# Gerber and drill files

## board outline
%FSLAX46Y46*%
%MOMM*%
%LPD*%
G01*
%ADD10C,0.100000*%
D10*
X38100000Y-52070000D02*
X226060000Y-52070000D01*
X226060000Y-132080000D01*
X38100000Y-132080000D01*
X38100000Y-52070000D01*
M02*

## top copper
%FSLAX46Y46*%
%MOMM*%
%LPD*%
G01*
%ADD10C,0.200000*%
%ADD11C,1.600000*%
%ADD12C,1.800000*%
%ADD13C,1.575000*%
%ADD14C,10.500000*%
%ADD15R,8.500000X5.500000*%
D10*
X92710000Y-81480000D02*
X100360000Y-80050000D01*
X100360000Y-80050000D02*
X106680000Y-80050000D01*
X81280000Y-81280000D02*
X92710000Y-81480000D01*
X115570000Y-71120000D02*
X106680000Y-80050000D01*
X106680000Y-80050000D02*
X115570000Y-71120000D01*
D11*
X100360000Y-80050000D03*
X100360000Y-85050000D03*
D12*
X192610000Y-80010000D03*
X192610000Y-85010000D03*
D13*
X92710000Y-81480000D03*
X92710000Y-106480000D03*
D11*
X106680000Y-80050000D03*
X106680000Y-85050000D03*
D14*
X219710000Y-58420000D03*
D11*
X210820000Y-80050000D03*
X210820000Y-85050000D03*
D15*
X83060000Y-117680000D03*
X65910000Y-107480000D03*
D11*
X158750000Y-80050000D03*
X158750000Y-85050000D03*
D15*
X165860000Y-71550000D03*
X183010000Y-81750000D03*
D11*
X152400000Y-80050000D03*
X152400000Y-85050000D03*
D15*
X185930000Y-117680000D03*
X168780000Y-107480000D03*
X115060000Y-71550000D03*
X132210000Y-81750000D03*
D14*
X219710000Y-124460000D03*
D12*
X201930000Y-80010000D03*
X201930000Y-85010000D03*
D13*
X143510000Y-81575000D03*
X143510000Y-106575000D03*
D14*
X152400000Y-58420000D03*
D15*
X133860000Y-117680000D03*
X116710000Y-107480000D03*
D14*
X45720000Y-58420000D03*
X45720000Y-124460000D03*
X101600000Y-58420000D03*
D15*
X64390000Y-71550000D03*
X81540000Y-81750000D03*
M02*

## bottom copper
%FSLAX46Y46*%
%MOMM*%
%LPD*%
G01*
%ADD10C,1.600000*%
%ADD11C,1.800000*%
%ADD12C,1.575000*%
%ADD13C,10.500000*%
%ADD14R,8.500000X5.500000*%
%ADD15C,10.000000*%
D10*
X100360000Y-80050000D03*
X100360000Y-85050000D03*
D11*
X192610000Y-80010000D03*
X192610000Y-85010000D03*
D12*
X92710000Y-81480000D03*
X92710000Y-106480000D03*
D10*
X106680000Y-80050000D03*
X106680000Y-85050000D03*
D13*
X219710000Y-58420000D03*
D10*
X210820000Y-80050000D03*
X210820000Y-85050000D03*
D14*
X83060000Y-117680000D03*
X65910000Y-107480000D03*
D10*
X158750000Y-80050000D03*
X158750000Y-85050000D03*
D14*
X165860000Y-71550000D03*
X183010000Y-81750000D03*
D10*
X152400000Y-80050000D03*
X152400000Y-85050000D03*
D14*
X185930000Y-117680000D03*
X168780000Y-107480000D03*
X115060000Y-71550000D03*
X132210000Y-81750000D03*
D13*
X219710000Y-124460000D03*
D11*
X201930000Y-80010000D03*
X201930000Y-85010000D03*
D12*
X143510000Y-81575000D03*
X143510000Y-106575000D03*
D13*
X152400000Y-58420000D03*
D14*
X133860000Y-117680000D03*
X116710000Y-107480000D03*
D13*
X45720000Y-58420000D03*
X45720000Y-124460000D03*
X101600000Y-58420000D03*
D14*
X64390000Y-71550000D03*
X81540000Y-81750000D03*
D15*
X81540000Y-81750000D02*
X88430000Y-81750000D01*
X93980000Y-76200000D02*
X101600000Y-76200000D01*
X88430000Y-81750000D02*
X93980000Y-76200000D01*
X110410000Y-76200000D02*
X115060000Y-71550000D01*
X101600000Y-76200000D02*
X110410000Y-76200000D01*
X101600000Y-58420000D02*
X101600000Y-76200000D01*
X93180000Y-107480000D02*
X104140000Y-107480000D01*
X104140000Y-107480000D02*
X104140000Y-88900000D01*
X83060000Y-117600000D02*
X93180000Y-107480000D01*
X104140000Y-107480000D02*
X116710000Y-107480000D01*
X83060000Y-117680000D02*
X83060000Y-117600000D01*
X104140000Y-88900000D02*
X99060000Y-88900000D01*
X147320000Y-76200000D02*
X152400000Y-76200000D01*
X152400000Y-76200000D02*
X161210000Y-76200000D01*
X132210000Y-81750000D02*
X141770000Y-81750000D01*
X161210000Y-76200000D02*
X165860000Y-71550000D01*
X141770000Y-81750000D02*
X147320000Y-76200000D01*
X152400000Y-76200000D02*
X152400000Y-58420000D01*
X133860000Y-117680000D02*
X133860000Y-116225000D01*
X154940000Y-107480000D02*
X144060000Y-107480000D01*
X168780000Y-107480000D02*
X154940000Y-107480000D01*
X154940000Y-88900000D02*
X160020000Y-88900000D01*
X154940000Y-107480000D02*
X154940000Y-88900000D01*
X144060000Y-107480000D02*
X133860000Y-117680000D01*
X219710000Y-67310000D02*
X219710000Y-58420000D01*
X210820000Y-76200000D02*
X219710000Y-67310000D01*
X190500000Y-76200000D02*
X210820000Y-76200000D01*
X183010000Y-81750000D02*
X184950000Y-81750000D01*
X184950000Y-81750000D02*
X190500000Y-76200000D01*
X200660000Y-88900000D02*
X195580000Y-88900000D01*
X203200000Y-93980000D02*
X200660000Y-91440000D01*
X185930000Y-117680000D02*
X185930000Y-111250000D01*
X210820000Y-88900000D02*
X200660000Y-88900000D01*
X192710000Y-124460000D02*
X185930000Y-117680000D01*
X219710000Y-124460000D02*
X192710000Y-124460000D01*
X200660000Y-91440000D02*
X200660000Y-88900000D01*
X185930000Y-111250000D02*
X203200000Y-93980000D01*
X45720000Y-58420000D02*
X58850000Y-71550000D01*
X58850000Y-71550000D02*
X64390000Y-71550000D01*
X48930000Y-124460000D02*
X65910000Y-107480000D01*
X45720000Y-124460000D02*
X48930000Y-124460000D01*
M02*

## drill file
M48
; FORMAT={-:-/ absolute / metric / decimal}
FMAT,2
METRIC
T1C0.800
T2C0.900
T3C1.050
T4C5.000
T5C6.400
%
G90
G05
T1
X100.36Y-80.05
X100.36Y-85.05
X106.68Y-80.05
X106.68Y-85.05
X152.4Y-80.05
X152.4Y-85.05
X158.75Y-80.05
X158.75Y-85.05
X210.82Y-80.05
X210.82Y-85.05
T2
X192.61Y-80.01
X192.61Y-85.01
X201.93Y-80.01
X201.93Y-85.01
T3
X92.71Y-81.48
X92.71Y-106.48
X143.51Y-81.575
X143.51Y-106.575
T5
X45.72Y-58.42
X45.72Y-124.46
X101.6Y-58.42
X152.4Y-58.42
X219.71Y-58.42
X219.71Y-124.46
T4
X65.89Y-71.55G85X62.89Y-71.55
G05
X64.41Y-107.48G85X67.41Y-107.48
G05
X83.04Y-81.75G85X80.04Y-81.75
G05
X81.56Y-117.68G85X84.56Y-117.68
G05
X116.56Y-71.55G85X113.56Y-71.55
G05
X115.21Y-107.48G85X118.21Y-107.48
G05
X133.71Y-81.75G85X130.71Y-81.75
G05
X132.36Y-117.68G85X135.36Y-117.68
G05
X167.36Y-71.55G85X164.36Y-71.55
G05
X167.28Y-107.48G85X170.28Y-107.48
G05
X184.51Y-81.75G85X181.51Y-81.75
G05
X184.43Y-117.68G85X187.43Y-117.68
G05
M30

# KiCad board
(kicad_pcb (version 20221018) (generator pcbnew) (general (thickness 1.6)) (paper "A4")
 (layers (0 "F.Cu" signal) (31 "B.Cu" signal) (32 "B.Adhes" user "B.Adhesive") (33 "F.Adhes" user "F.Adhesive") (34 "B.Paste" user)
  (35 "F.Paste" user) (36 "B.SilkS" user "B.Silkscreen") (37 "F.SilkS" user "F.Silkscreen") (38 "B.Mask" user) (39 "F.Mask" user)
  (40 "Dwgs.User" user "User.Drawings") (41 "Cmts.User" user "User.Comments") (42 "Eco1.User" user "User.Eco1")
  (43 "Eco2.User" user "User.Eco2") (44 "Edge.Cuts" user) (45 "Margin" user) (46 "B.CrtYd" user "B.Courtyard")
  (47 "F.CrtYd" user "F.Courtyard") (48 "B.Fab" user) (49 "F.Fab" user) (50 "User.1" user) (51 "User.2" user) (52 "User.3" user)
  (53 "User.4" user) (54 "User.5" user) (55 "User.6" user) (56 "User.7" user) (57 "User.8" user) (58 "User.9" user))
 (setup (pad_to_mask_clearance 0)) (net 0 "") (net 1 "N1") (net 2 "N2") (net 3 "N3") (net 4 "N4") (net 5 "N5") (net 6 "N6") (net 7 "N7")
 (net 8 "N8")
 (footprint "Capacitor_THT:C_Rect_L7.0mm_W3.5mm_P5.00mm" (layer "F.Cu") (at 100.36 80.05 -90)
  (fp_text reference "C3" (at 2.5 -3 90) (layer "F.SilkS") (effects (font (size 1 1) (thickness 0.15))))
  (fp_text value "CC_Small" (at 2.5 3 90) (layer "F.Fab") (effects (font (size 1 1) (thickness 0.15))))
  (pad "1" thru_hole circle (at 0 0 270) (size 1.6 1.6) (drill 0.8) (layers "*.Cu" "*.Mask") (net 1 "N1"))
  (pad "2" thru_hole circle (at 5 0 270) (size 1.6 1.6) (drill 0.8) (layers "*.Cu" "*.Mask") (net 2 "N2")))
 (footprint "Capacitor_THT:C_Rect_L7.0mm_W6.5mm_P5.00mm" (layer "F.Cu") (at 192.61 80.01 -90)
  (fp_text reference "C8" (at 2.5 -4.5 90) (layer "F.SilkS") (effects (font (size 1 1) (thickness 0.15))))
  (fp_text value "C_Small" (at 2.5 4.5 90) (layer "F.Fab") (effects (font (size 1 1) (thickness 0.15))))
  (pad "1" thru_hole circle (at 0 0 270) (size 1.8 1.8) (drill 0.9) (layers "*.Cu" "*.Mask") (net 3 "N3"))
  (pad "2" thru_hole circle (at 5 0 270) (size 1.8 1.8) (drill 0.9) (layers "*.Cu" "*.Mask") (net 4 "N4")))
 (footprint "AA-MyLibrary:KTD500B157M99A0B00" (layer "F.Cu") (at 92.71 81.48 -90)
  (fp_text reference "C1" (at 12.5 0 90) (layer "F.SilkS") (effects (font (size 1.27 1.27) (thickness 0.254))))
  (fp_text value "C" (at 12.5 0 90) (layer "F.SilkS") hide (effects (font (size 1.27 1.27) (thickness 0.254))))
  (pad "1" thru_hole circle (at 0 0 270) (size 1.575 1.575) (drill 1.05) (layers "*.Cu" "*.Mask") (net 1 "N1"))
  (pad "2" thru_hole circle (at 25 0 270) (size 1.575 1.575) (drill 1.05) (layers "*.Cu" "*.Mask") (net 2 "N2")))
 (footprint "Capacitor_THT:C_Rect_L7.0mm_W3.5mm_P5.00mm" (layer "F.Cu") (at 106.68 80.05 -90)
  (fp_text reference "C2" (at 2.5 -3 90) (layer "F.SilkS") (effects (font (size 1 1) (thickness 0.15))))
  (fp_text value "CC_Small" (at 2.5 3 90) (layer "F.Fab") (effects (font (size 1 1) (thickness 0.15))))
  (pad "1" thru_hole circle (at 0 0 270) (size 1.6 1.6) (drill 0.8) (layers "*.Cu" "*.Mask") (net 1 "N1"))
  (pad "2" thru_hole circle (at 5 0 270) (size 1.6 1.6) (drill 0.8) (layers "*.Cu" "*.Mask") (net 2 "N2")))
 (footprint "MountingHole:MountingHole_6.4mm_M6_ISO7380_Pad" (layer "F.Cu") (at 219.71 58.42)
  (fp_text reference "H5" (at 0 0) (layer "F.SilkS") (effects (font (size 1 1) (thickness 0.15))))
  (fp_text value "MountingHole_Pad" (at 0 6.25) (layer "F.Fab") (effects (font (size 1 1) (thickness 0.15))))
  (pad "1" thru_hole circle (at 0 0) (size 10.5 10.5) (drill 6.4) (layers "*.Cu" "*.Mask") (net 3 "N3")))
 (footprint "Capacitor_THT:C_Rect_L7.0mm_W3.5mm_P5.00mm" (layer "F.Cu") (at 210.82 80.05 -90)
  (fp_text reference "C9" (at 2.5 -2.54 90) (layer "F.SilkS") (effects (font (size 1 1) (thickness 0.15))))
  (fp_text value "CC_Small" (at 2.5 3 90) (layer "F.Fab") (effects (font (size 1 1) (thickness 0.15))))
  (pad "1" thru_hole circle (at 0 0 270) (size 1.6 1.6) (drill 0.8) (layers "*.Cu" "*.Mask") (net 3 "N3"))
  (pad "2" thru_hole circle (at 5 0 270) (size 1.6 1.6) (drill 0.8) (layers "*.Cu" "*.Mask") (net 4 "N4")))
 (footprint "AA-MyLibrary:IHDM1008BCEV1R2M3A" (layer "F.Cu") (at 73.66 113.03)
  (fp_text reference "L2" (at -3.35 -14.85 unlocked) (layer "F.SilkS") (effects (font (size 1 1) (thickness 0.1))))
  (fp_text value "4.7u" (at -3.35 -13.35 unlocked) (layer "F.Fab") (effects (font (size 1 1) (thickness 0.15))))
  (pad "1" thru_hole rect (at 9.4 4.65) (size 8.5 5.5) (drill oval 8 5) (layers "*.Cu" "*.Mask") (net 2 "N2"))
  (pad "2" thru_hole rect (at -7.75 -5.55) (size 8.5 5.5) (drill oval 8 5) (layers "*.Cu" "*.Mask") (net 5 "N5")))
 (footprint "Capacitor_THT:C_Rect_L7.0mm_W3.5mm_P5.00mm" (layer "F.Cu") (at 158.75 80.05 -90)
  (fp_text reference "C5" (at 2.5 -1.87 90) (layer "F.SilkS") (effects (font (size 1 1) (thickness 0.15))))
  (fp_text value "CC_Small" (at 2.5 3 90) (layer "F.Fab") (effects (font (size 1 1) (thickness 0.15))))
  (pad "1" thru_hole circle (at 0 0 270) (size 1.6 1.6) (drill 0.8) (layers "*.Cu" "*.Mask") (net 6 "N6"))
  (pad "2" thru_hole circle (at 5 0 270) (size 1.6 1.6) (drill 0.8) (layers "*.Cu" "*.Mask") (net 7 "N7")))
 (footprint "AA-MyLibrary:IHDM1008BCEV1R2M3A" (layer "F.Cu") (at 175.26 76.2 180)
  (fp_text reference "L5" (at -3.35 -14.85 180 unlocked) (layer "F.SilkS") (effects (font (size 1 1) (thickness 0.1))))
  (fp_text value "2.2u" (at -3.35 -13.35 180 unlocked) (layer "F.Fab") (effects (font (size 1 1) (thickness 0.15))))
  (pad "1" thru_hole rect (at 9.4 4.65 180) (size 8.5 5.5) (drill oval 8 5) (layers "*.Cu" "*.Mask") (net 6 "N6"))
  (pad "2" thru_hole rect (at -7.75 -5.55 180) (size 8.5 5.5) (drill oval 8 5) (layers "*.Cu" "*.Mask") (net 3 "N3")))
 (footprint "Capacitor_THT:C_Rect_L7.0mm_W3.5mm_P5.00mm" (layer "F.Cu") (at 152.4 80.05 -90)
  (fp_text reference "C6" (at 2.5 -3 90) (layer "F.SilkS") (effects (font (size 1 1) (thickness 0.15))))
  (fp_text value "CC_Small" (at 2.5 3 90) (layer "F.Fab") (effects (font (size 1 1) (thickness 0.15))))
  (pad "1" thru_hole circle (at 0 0 270) (size 1.6 1.6) (drill 0.8) (layers "*.Cu" "*.Mask") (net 6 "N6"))
  (pad "2" thru_hole circle (at 5 0 270) (size 1.6 1.6) (drill 0.8) (layers "*.Cu" "*.Mask") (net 7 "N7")))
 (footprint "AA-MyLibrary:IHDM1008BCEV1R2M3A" (layer "F.Cu") (at 176.53 113.03)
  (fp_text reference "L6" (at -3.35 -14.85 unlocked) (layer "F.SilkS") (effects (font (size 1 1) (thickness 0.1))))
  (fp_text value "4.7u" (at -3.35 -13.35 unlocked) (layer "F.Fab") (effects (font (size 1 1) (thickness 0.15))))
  (pad "1" thru_hole rect (at 9.4 4.65) (size 8.5 5.5) (drill oval 8 5) (layers "*.Cu" "*.Mask") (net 4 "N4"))
  (pad "2" thru_hole rect (at -7.75 -5.55) (size 8.5 5.5) (drill oval 8 5) (layers "*.Cu" "*.Mask") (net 7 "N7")))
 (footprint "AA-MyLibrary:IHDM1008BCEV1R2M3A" (layer "F.Cu") (at 124.46 76.2 180)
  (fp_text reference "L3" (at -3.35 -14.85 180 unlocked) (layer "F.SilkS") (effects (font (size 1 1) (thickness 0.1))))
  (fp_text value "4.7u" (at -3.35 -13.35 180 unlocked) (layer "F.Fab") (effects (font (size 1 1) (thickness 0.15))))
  (pad "1" thru_hole rect (at 9.4 4.65 180) (size 8.5 5.5) (drill oval 8 5) (layers "*.Cu" "*.Mask") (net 1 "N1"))
  (pad "2" thru_hole rect (at -7.75 -5.55 180) (size 8.5 5.5) (drill oval 8 5) (layers "*.Cu" "*.Mask") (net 6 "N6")))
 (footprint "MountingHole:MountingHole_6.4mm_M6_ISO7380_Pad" (layer "F.Cu") (at 219.71 124.46)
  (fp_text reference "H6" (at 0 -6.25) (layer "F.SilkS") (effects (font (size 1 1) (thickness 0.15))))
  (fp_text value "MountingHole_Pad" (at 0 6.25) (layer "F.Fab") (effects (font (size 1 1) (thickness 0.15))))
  (pad "1" thru_hole circle (at 0 0) (size 10.5 10.5) (drill 6.4) (layers "*.Cu" "*.Mask") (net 4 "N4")))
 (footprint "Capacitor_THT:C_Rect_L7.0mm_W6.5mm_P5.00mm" (layer "F.Cu") (at 201.93 80.01 -90)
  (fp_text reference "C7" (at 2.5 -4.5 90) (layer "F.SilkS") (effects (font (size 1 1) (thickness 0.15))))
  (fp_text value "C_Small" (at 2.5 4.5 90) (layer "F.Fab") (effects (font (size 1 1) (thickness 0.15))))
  (pad "1" thru_hole circle (at 0 0 270) (size 1.8 1.8) (drill 0.9) (layers "*.Cu" "*.Mask") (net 3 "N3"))
  (pad "2" thru_hole circle (at 5 0 270) (size 1.8 1.8) (drill 0.9) (layers "*.Cu" "*.Mask") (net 4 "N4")))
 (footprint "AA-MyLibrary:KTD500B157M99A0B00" (layer "F.Cu") (at 143.51 81.575 -90)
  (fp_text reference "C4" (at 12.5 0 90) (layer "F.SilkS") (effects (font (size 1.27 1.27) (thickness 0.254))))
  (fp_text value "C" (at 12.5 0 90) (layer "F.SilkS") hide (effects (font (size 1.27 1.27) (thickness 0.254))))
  (pad "1" thru_hole circle (at 0 0 270) (size 1.575 1.575) (drill 1.05) (layers "*.Cu" "*.Mask") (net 6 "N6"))
  (pad "2" thru_hole circle (at 25 0 270) (size 1.575 1.575) (drill 1.05) (layers "*.Cu" "*.Mask") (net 7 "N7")))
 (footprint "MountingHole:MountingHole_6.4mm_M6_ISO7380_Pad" (layer "F.Cu") (at 152.4 58.42)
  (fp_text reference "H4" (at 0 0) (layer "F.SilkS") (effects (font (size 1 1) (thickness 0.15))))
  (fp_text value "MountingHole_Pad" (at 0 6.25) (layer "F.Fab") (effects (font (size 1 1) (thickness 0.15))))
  (pad "1" thru_hole circle (at 0 0) (size 10.5 10.5) (drill 6.4) (layers "*.Cu" "*.Mask") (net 6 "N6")))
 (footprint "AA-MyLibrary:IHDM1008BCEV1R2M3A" (layer "F.Cu") (at 124.46 113.03)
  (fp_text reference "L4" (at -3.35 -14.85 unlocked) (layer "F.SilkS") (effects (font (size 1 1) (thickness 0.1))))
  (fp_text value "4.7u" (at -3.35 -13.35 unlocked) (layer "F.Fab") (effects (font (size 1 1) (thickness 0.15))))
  (pad "1" thru_hole rect (at 9.4 4.65) (size 8.5 5.5) (drill oval 8 5) (layers "*.Cu" "*.Mask") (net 7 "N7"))
  (pad "2" thru_hole rect (at -7.75 -5.55) (size 8.5 5.5) (drill oval 8 5) (layers "*.Cu" "*.Mask") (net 2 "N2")))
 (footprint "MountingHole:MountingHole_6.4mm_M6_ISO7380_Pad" (layer "F.Cu") (at 45.72 58.42)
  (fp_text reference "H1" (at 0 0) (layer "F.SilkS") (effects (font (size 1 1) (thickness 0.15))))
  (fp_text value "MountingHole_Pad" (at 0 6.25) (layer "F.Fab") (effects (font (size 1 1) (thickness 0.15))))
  (pad "1" thru_hole circle (at 0 0) (size 10.5 10.5) (drill 6.4) (layers "*.Cu" "*.Mask") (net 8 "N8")))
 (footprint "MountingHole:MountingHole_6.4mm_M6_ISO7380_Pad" (layer "F.Cu") (at 45.72 124.46)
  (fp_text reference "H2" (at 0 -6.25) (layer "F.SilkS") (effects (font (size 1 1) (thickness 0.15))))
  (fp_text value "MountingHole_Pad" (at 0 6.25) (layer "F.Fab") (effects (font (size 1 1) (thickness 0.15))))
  (pad "1" thru_hole circle (at 0 0) (size 10.5 10.5) (drill 6.4) (layers "*.Cu" "*.Mask") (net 5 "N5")))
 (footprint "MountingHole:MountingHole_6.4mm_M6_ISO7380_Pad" (layer "F.Cu") (at 101.6 58.42)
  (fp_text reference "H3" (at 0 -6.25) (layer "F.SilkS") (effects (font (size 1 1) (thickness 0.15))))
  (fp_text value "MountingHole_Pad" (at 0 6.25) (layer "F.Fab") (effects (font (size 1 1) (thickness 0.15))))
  (pad "1" thru_hole circle (at 0 0) (size 10.5 10.5) (drill 6.4) (layers "*.Cu" "*.Mask") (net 1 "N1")))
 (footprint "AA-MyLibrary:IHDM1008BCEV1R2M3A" (layer "F.Cu") (at 73.79 76.2 180)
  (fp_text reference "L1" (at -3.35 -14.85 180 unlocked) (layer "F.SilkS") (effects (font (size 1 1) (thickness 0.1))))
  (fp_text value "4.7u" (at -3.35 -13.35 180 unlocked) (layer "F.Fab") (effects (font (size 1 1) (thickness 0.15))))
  (pad "1" thru_hole rect (at 9.4 4.65 180) (size 8.5 5.5) (drill oval 8 5) (layers "*.Cu" "*.Mask") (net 8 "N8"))
  (pad "2" thru_hole rect (at -7.75 -5.55 180) (size 8.5 5.5) (drill oval 8 5) (layers "*.Cu" "*.Mask") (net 1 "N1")))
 (gr_line (start 92.71 81.48) (end 100.36 80.05) (stroke (width 0.2) (type default)) (layer "F.Cu"))
 (gr_line (start 100.36 80.05) (end 106.68 80.05) (stroke (width 0.2) (type default)) (layer "F.Cu"))
 (gr_line (start 81.28 81.28) (end 92.71 81.48) (stroke (width 0.2) (type default)) (layer "F.Cu"))
 (gr_line (start 115.57 71.12) (end 106.68 80.05) (stroke (width 0.2) (type default)) (layer "F.Cu"))
 (gr_line (start 106.68 80.05) (end 115.57 71.12) (stroke (width 0.2) (type default)) (layer "F.Cu"))
 (gr_rect (start 38.1 52.07) (end 226.06 132.08) (stroke (width 0.1) (type default)) (fill none) (layer "Edge.Cuts"))
 (segment (start 81.54 81.75) (end 88.43 81.75) (width 10) (layer "B.Cu") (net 1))
 (segment (start 93.98 76.2) (end 101.6 76.2) (width 10) (layer "B.Cu") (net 1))
 (segment (start 88.43 81.75) (end 93.98 76.2) (width 10) (layer "B.Cu") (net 1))
 (segment (start 110.41 76.2) (end 115.06 71.55) (width 10) (layer "B.Cu") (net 1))
 (segment (start 101.6 76.2) (end 110.41 76.2) (width 10) (layer "B.Cu") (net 1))
 (segment (start 101.6 58.42) (end 101.6 76.2) (width 10) (layer "B.Cu") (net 1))
 (segment (start 93.18 107.48) (end 104.14 107.48) (width 10) (layer "B.Cu") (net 2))
 (segment (start 104.14 107.48) (end 104.14 88.9) (width 10) (layer "B.Cu") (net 2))
 (segment (start 83.06 117.6) (end 93.18 107.48) (width 10) (layer "B.Cu") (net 2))
 (segment (start 104.14 107.48) (end 116.71 107.48) (width 10) (layer "B.Cu") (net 2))
 (segment (start 83.06 117.68) (end 83.06 117.6) (width 10) (layer "B.Cu") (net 2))
 (segment (start 104.14 88.9) (end 99.06 88.9) (width 10) (layer "B.Cu") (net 2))
 (segment (start 147.32 76.2) (end 152.4 76.2) (width 10) (layer "B.Cu") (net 6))
 (segment (start 152.4 76.2) (end 161.21 76.2) (width 10) (layer "B.Cu") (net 6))
 (segment (start 132.21 81.75) (end 141.77 81.75) (width 10) (layer "B.Cu") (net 6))
 (segment (start 161.21 76.2) (end 165.86 71.55) (width 10) (layer "B.Cu") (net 6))
 (segment (start 141.77 81.75) (end 147.32 76.2) (width 10) (layer "B.Cu") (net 6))
 (segment (start 152.4 76.2) (end 152.4 58.42) (width 10) (layer "B.Cu") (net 6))
 (segment (start 133.86 117.68) (end 133.86 116.225) (width 10) (layer "B.Cu") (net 7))
 (segment (start 154.94 107.48) (end 144.06 107.48) (width 10) (layer "B.Cu") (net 7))
 (segment (start 168.78 107.48) (end 154.94 107.48) (width 10) (layer "B.Cu") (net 7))
 (segment (start 154.94 88.9) (end 160.02 88.9) (width 10) (layer "B.Cu") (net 7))
 (segment (start 154.94 107.48) (end 154.94 88.9) (width 10) (layer "B.Cu") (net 7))
 (segment (start 144.06 107.48) (end 133.86 117.68) (width 10) (layer "B.Cu") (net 7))
 (segment (start 219.71 67.31) (end 219.71 58.42) (width 10) (layer "B.Cu") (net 3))
 (segment (start 210.82 76.2) (end 219.71 67.31) (width 10) (layer "B.Cu") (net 3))
 (segment (start 190.5 76.2) (end 210.82 76.2) (width 10) (layer "B.Cu") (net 3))
 (segment (start 183.01 81.75) (end 184.95 81.75) (width 10) (layer "B.Cu") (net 3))
 (segment (start 184.95 81.75) (end 190.5 76.2) (width 10) (layer "B.Cu") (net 3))
 (segment (start 200.66 88.9) (end 195.58 88.9) (width 10) (layer "B.Cu") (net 4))
 (segment (start 203.2 93.98) (end 200.66 91.44) (width 10) (layer "B.Cu") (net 4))
 (segment (start 185.93 117.68) (end 185.93 111.25) (width 10) (layer "B.Cu") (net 4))
 (segment (start 210.82 88.9) (end 200.66 88.9) (width 10) (layer "B.Cu") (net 4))
 (segment (start 192.71 124.46) (end 185.93 117.68) (width 10) (layer "B.Cu") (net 4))
 (segment (start 219.71 124.46) (end 192.71 124.46) (width 10) (layer "B.Cu") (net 4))
 (segment (start 200.66 91.44) (end 200.66 88.9) (width 10) (layer "B.Cu") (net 4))
 (segment (start 185.93 111.25) (end 203.2 93.98) (width 10) (layer "B.Cu") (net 4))
 (segment (start 45.72 58.42) (end 58.85 71.55) (width 10) (layer "B.Cu") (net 8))
 (segment (start 58.85 71.55) (end 64.39 71.55) (width 10) (layer "B.Cu") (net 8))
 (segment (start 48.93 124.46) (end 65.91 107.48) (width 10) (layer "B.Cu") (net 5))
 (segment (start 45.72 124.46) (end 48.93 124.46) (width 10) (layer "B.Cu") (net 5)))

